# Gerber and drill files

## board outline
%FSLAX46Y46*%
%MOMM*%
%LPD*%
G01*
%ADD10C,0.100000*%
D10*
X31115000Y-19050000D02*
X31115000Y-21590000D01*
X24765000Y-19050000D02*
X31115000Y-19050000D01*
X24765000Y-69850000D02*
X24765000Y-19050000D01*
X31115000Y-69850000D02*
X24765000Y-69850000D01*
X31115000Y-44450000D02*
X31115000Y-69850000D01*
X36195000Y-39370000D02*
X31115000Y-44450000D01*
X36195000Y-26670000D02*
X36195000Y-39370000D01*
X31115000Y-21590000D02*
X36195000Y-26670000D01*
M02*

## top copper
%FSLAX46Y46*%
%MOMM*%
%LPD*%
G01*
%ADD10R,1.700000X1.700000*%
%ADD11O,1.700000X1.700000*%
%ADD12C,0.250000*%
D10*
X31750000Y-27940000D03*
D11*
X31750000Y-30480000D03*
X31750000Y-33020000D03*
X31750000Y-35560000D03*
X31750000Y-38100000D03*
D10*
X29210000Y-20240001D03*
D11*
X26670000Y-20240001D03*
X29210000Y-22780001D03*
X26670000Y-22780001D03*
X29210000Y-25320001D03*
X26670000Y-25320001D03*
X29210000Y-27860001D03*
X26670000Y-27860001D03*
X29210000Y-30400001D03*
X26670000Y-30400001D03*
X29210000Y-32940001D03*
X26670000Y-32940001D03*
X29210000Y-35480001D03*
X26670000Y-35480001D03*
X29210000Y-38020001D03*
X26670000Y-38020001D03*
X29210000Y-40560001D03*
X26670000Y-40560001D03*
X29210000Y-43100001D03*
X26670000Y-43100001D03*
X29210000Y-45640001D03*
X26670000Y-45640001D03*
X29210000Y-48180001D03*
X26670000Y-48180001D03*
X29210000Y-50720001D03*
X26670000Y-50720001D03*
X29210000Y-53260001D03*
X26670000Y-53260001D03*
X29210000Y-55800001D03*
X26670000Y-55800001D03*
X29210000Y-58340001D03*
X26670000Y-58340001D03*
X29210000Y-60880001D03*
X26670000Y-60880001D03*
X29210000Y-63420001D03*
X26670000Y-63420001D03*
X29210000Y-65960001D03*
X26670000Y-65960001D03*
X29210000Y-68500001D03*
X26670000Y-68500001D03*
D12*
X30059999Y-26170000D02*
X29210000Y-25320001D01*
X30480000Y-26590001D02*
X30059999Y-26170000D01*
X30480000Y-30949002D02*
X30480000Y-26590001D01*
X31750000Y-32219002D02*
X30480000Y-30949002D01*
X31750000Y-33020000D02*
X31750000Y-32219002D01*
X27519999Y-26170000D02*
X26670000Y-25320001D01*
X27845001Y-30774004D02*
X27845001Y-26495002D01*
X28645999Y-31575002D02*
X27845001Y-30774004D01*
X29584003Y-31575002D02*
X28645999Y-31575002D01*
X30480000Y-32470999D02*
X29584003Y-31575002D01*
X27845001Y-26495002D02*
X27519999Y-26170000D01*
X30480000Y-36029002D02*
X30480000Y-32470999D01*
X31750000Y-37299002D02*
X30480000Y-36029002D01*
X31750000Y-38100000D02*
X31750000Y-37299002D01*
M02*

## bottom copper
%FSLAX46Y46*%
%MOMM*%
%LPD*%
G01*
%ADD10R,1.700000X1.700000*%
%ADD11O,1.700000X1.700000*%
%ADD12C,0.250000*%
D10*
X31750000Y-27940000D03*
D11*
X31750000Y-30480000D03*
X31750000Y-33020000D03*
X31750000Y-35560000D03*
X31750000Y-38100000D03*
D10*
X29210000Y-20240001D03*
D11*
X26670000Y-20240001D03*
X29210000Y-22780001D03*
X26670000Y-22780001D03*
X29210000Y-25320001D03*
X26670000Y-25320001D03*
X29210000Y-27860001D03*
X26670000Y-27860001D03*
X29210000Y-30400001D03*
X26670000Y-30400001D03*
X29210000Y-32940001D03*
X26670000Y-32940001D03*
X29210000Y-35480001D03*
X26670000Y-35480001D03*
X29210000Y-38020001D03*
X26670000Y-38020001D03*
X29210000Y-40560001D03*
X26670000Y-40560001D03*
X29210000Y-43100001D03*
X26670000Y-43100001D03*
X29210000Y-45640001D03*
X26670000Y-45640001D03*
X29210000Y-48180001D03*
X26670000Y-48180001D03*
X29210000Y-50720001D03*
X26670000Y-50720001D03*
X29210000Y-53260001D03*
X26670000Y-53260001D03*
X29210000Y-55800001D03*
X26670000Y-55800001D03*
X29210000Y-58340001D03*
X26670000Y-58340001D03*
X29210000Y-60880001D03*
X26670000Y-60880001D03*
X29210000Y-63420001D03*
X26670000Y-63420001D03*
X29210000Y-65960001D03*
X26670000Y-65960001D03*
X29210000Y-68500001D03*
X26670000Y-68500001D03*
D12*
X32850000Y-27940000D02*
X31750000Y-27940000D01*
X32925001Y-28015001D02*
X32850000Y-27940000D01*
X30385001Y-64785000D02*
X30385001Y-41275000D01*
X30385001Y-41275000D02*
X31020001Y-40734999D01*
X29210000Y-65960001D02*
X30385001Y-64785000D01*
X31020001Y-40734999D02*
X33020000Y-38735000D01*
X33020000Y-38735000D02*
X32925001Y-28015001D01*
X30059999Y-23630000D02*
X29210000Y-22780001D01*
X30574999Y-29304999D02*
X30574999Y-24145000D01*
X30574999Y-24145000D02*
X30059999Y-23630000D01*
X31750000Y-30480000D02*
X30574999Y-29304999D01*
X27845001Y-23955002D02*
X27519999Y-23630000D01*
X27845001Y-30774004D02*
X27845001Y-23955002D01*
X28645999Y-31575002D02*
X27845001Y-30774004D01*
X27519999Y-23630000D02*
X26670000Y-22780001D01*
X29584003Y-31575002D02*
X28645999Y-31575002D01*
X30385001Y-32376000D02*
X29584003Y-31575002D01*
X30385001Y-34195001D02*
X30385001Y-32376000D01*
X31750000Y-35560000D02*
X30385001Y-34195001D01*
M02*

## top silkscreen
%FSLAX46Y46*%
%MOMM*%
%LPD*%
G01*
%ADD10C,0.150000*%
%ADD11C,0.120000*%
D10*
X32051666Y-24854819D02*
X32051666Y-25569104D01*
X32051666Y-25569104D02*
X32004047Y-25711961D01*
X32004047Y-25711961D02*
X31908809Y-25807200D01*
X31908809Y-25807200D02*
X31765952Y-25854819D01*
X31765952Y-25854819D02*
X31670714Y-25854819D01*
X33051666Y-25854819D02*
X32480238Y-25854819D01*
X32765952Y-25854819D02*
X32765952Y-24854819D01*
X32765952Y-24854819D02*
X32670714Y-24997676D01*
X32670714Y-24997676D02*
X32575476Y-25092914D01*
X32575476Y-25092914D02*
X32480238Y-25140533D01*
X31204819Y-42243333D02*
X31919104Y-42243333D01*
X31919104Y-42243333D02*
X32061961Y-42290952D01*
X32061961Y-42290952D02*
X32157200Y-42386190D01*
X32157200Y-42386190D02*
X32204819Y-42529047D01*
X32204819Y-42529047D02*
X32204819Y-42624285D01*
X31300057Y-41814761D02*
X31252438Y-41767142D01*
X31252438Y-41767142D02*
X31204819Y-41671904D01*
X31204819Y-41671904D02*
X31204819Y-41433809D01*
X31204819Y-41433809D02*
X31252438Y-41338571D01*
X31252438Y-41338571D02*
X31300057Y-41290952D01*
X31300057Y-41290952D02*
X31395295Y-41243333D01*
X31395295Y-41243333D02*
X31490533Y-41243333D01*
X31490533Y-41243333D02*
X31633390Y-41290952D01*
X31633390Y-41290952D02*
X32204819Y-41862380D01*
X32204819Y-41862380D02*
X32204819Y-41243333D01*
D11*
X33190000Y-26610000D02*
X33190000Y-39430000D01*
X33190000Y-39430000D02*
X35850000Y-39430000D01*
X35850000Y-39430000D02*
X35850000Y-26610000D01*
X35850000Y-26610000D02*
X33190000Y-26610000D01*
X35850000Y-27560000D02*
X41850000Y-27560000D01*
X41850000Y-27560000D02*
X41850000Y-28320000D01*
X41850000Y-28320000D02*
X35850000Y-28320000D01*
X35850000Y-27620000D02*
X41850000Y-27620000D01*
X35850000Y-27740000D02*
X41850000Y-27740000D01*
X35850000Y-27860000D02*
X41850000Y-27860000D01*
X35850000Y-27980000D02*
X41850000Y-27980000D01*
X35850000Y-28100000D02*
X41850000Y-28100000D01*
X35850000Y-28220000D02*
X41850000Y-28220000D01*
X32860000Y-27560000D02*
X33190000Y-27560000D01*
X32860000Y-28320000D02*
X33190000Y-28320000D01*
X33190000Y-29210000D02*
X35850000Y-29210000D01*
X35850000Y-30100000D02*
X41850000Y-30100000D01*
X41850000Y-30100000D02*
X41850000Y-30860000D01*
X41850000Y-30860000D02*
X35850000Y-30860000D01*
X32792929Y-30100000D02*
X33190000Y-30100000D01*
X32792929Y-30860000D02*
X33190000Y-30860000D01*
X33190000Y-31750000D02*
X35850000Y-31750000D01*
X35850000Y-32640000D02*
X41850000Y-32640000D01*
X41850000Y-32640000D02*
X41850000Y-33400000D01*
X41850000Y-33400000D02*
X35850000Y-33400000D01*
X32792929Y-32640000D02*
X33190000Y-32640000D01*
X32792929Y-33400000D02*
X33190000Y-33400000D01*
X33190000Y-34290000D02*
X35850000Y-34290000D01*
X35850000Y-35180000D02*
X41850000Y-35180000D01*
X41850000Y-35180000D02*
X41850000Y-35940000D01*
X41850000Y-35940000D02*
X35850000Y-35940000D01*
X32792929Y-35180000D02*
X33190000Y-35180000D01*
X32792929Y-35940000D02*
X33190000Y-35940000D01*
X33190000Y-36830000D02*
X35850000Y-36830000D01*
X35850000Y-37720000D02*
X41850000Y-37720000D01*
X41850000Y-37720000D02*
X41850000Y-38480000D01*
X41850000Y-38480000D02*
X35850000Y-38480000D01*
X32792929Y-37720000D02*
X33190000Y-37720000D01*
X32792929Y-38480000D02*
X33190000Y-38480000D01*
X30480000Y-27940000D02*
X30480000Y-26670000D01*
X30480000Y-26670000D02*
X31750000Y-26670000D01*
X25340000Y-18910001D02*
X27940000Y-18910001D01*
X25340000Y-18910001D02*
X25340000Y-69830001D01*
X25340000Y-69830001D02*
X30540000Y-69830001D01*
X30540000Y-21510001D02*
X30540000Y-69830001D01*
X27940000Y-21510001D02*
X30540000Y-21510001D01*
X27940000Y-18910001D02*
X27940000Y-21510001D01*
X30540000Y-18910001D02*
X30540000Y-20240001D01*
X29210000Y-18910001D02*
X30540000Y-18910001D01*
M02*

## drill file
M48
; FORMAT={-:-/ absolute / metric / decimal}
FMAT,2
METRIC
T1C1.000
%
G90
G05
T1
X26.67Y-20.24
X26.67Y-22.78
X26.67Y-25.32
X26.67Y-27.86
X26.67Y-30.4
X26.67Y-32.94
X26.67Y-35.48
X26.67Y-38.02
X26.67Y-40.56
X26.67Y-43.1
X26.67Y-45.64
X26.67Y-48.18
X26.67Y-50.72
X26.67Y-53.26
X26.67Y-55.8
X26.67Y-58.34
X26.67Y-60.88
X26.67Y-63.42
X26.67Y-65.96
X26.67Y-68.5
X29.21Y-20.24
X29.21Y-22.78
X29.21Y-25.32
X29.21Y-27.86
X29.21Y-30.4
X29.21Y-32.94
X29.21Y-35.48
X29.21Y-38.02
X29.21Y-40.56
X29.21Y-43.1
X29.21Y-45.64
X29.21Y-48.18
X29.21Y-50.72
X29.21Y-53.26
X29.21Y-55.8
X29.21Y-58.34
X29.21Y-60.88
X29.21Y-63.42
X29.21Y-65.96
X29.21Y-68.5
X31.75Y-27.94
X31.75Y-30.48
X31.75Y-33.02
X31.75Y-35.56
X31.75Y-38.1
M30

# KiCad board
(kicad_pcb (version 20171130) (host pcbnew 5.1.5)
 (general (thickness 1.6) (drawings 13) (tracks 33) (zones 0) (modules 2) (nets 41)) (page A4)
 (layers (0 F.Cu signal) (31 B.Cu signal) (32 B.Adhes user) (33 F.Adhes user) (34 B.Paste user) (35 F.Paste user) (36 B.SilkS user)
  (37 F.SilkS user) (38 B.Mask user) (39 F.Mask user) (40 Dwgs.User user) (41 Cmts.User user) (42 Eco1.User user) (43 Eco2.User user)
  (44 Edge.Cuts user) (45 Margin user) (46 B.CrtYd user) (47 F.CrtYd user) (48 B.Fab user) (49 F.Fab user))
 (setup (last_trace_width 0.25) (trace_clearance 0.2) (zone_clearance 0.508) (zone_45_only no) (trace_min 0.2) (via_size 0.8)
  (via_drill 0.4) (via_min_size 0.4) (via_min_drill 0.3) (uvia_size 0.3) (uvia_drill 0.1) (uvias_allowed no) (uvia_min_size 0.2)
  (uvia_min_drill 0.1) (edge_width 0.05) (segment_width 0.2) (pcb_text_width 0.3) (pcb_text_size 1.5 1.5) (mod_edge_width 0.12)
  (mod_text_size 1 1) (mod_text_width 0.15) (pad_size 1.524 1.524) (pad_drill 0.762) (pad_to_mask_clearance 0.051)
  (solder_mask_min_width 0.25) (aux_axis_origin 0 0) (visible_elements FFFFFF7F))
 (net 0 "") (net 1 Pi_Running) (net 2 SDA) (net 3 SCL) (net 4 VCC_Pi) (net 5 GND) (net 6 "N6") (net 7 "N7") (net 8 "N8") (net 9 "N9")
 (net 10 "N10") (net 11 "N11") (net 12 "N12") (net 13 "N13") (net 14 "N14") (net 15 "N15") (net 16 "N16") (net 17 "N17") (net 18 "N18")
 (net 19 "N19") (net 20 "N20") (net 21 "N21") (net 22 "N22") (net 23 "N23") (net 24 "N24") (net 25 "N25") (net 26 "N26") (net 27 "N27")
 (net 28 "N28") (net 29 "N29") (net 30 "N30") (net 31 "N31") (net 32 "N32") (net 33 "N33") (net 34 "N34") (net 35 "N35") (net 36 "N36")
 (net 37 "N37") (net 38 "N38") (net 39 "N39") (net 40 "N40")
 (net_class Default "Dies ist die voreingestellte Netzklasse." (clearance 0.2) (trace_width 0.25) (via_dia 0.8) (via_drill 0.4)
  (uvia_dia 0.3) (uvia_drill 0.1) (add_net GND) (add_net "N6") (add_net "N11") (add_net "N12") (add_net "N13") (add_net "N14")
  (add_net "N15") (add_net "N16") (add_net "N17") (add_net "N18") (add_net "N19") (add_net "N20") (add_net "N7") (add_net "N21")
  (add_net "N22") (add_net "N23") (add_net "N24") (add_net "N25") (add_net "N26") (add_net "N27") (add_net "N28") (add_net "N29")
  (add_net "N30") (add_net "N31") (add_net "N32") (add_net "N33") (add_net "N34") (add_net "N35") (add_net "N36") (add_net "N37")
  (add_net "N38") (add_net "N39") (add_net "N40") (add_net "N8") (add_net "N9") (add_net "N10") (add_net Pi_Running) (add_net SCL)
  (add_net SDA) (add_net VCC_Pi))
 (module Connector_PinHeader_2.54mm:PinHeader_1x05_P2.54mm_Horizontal (layer F.Cu) (at 31.75 27.94)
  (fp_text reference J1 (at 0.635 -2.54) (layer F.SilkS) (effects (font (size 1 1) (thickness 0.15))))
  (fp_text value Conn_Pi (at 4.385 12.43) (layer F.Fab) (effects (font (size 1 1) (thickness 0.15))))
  (fp_line (start 1.44 -1.33) (end 1.44 11.49) (layer F.SilkS) (width 0.12))
  (fp_line (start 1.44 11.49) (end 4.1 11.49) (layer F.SilkS) (width 0.12))
  (fp_line (start 4.1 11.49) (end 4.1 -1.33) (layer F.SilkS) (width 0.12))
  (fp_line (start 4.1 -1.33) (end 1.44 -1.33) (layer F.SilkS) (width 0.12))
  (fp_line (start 4.1 -0.38) (end 10.1 -0.38) (layer F.SilkS) (width 0.12))
  (fp_line (start 10.1 -0.38) (end 10.1 0.38) (layer F.SilkS) (width 0.12))
  (fp_line (start 10.1 0.38) (end 4.1 0.38) (layer F.SilkS) (width 0.12))
  (fp_line (start 4.1 -0.32) (end 10.1 -0.32) (layer F.SilkS) (width 0.12))
  (fp_line (start 4.1 -0.2) (end 10.1 -0.2) (layer F.SilkS) (width 0.12))
  (fp_line (start 4.1 -0.08) (end 10.1 -0.08) (layer F.SilkS) (width 0.12))
  (fp_line (start 4.1 0.04) (end 10.1 0.04) (layer F.SilkS) (width 0.12))
  (fp_line (start 4.1 0.16) (end 10.1 0.16) (layer F.SilkS) (width 0.12))
  (fp_line (start 4.1 0.28) (end 10.1 0.28) (layer F.SilkS) (width 0.12))
  (fp_line (start 1.11 -0.38) (end 1.44 -0.38) (layer F.SilkS) (width 0.12))
  (fp_line (start 1.11 0.38) (end 1.44 0.38) (layer F.SilkS) (width 0.12))
  (fp_line (start 1.44 1.27) (end 4.1 1.27) (layer F.SilkS) (width 0.12))
  (fp_line (start 4.1 2.16) (end 10.1 2.16) (layer F.SilkS) (width 0.12))
  (fp_line (start 10.1 2.16) (end 10.1 2.92) (layer F.SilkS) (width 0.12))
  (fp_line (start 10.1 2.92) (end 4.1 2.92) (layer F.SilkS) (width 0.12))
  (fp_line (start 1.042929 2.16) (end 1.44 2.16) (layer F.SilkS) (width 0.12))
  (fp_line (start 1.042929 2.92) (end 1.44 2.92) (layer F.SilkS) (width 0.12))
  (fp_line (start 1.44 3.81) (end 4.1 3.81) (layer F.SilkS) (width 0.12))
  (fp_line (start 4.1 4.7) (end 10.1 4.7) (layer F.SilkS) (width 0.12))
  (fp_line (start 10.1 4.7) (end 10.1 5.46) (layer F.SilkS) (width 0.12))
  (fp_line (start 10.1 5.46) (end 4.1 5.46) (layer F.SilkS) (width 0.12))
  (fp_line (start 1.042929 4.7) (end 1.44 4.7) (layer F.SilkS) (width 0.12))
  (fp_line (start 1.042929 5.46) (end 1.44 5.46) (layer F.SilkS) (width 0.12))
  (fp_line (start 1.44 6.35) (end 4.1 6.35) (layer F.SilkS) (width 0.12))
  (fp_line (start 4.1 7.24) (end 10.1 7.24) (layer F.SilkS) (width 0.12))
  (fp_line (start 10.1 7.24) (end 10.1 8) (layer F.SilkS) (width 0.12))
  (fp_line (start 10.1 8) (end 4.1 8) (layer F.SilkS) (width 0.12))
  (fp_line (start 1.042929 7.24) (end 1.44 7.24) (layer F.SilkS) (width 0.12))
  (fp_line (start 1.042929 8) (end 1.44 8) (layer F.SilkS) (width 0.12))
  (fp_line (start 1.44 8.89) (end 4.1 8.89) (layer F.SilkS) (width 0.12))
  (fp_line (start 4.1 9.78) (end 10.1 9.78) (layer F.SilkS) (width 0.12))
  (fp_line (start 10.1 9.78) (end 10.1 10.54) (layer F.SilkS) (width 0.12))
  (fp_line (start 10.1 10.54) (end 4.1 10.54) (layer F.SilkS) (width 0.12))
  (fp_line (start 1.042929 9.78) (end 1.44 9.78) (layer F.SilkS) (width 0.12))
  (fp_line (start 1.042929 10.54) (end 1.44 10.54) (layer F.SilkS) (width 0.12))
  (fp_line (start -1.27 0) (end -1.27 -1.27) (layer F.SilkS) (width 0.12))
  (fp_line (start -1.27 -1.27) (end 0 -1.27) (layer F.SilkS) (width 0.12))
  (pad 1 thru_hole rect (at 0 0) (size 1.7 1.7) (drill 1) (layers *.Cu *.Mask) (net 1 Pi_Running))
  (pad 2 thru_hole oval (at 0 2.54) (size 1.7 1.7) (drill 1) (layers *.Cu *.Mask) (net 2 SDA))
  (pad 3 thru_hole oval (at 0 5.08) (size 1.7 1.7) (drill 1) (layers *.Cu *.Mask) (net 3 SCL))
  (pad 4 thru_hole oval (at 0 7.62) (size 1.7 1.7) (drill 1) (layers *.Cu *.Mask) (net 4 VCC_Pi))
  (pad 5 thru_hole oval (at 0 10.16) (size 1.7 1.7) (drill 1) (layers *.Cu *.Mask) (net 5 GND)))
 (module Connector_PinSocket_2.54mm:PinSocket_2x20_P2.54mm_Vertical (layer F.Cu) (at 29.21 20.240001)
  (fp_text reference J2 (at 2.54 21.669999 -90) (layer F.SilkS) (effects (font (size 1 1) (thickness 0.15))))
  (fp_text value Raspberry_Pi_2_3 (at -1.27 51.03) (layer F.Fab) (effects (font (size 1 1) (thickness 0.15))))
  (fp_line (start -3.87 -1.33) (end -1.27 -1.33) (layer F.SilkS) (width 0.12))
  (fp_line (start -3.87 -1.33) (end -3.87 49.59) (layer F.SilkS) (width 0.12))
  (fp_line (start -3.87 49.59) (end 1.33 49.59) (layer F.SilkS) (width 0.12))
  (fp_line (start 1.33 1.27) (end 1.33 49.59) (layer F.SilkS) (width 0.12))
  (fp_line (start -1.27 1.27) (end 1.33 1.27) (layer F.SilkS) (width 0.12))
  (fp_line (start -1.27 -1.33) (end -1.27 1.27) (layer F.SilkS) (width 0.12))
  (fp_line (start 1.33 -1.33) (end 1.33 0) (layer F.SilkS) (width 0.12))
  (fp_line (start 0 -1.33) (end 1.33 -1.33) (layer F.SilkS) (width 0.12))
  (pad 1 thru_hole rect (at 0 0) (size 1.7 1.7) (drill 1) (layers *.Cu *.Mask) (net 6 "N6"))
  (pad 2 thru_hole oval (at -2.54 0) (size 1.7 1.7) (drill 1) (layers *.Cu *.Mask) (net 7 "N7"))
  (pad 3 thru_hole oval (at 0 2.54) (size 1.7 1.7) (drill 1) (layers *.Cu *.Mask) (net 2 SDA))
  (pad 4 thru_hole oval (at -2.54 2.54) (size 1.7 1.7) (drill 1) (layers *.Cu *.Mask) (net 4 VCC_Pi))
  (pad 5 thru_hole oval (at 0 5.08) (size 1.7 1.7) (drill 1) (layers *.Cu *.Mask) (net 3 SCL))
  (pad 6 thru_hole oval (at -2.54 5.08) (size 1.7 1.7) (drill 1) (layers *.Cu *.Mask) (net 5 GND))
  (pad 7 thru_hole oval (at 0 7.62) (size 1.7 1.7) (drill 1) (layers *.Cu *.Mask) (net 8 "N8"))
  (pad 8 thru_hole oval (at -2.54 7.62) (size 1.7 1.7) (drill 1) (layers *.Cu *.Mask) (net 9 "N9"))
  (pad 9 thru_hole oval (at 0 10.16) (size 1.7 1.7) (drill 1) (layers *.Cu *.Mask) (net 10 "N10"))
  (pad 10 thru_hole oval (at -2.54 10.16) (size 1.7 1.7) (drill 1) (layers *.Cu *.Mask) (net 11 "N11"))
  (pad 11 thru_hole oval (at 0 12.7) (size 1.7 1.7) (drill 1) (layers *.Cu *.Mask) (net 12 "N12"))
  (pad 12 thru_hole oval (at -2.54 12.7) (size 1.7 1.7) (drill 1) (layers *.Cu *.Mask) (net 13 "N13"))
  (pad 13 thru_hole oval (at 0 15.24) (size 1.7 1.7) (drill 1) (layers *.Cu *.Mask) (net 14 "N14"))
  (pad 14 thru_hole oval (at -2.54 15.24) (size 1.7 1.7) (drill 1) (layers *.Cu *.Mask) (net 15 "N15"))
  (pad 15 thru_hole oval (at 0 17.78) (size 1.7 1.7) (drill 1) (layers *.Cu *.Mask) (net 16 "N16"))
  (pad 16 thru_hole oval (at -2.54 17.78) (size 1.7 1.7) (drill 1) (layers *.Cu *.Mask) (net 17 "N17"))
  (pad 17 thru_hole oval (at 0 20.32) (size 1.7 1.7) (drill 1) (layers *.Cu *.Mask) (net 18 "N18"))
  (pad 18 thru_hole oval (at -2.54 20.32) (size 1.7 1.7) (drill 1) (layers *.Cu *.Mask) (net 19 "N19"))
  (pad 19 thru_hole oval (at 0 22.86) (size 1.7 1.7) (drill 1) (layers *.Cu *.Mask) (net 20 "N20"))
  (pad 20 thru_hole oval (at -2.54 22.86) (size 1.7 1.7) (drill 1) (layers *.Cu *.Mask) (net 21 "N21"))
  (pad 21 thru_hole oval (at 0 25.4) (size 1.7 1.7) (drill 1) (layers *.Cu *.Mask) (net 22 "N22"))
  (pad 22 thru_hole oval (at -2.54 25.4) (size 1.7 1.7) (drill 1) (layers *.Cu *.Mask) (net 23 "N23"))
  (pad 23 thru_hole oval (at 0 27.94) (size 1.7 1.7) (drill 1) (layers *.Cu *.Mask) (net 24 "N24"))
  (pad 24 thru_hole oval (at -2.54 27.94) (size 1.7 1.7) (drill 1) (layers *.Cu *.Mask) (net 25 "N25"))
  (pad 25 thru_hole oval (at 0 30.48) (size 1.7 1.7) (drill 1) (layers *.Cu *.Mask) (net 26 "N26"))
  (pad 26 thru_hole oval (at -2.54 30.48) (size 1.7 1.7) (drill 1) (layers *.Cu *.Mask) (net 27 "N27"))
  (pad 27 thru_hole oval (at 0 33.02) (size 1.7 1.7) (drill 1) (layers *.Cu *.Mask) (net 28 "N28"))
  (pad 28 thru_hole oval (at -2.54 33.02) (size 1.7 1.7) (drill 1) (layers *.Cu *.Mask) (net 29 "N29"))
  (pad 29 thru_hole oval (at 0 35.56) (size 1.7 1.7) (drill 1) (layers *.Cu *.Mask) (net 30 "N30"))
  (pad 30 thru_hole oval (at -2.54 35.56) (size 1.7 1.7) (drill 1) (layers *.Cu *.Mask) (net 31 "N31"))
  (pad 31 thru_hole oval (at 0 38.1) (size 1.7 1.7) (drill 1) (layers *.Cu *.Mask) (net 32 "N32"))
  (pad 32 thru_hole oval (at -2.54 38.1) (size 1.7 1.7) (drill 1) (layers *.Cu *.Mask) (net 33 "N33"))
  (pad 33 thru_hole oval (at 0 40.64) (size 1.7 1.7) (drill 1) (layers *.Cu *.Mask) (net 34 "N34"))
  (pad 34 thru_hole oval (at -2.54 40.64) (size 1.7 1.7) (drill 1) (layers *.Cu *.Mask) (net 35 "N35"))
  (pad 35 thru_hole oval (at 0 43.18) (size 1.7 1.7) (drill 1) (layers *.Cu *.Mask) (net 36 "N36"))
  (pad 36 thru_hole oval (at -2.54 43.18) (size 1.7 1.7) (drill 1) (layers *.Cu *.Mask) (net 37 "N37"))
  (pad 37 thru_hole oval (at 0 45.72) (size 1.7 1.7) (drill 1) (layers *.Cu *.Mask) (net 1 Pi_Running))
  (pad 38 thru_hole oval (at -2.54 45.72) (size 1.7 1.7) (drill 1) (layers *.Cu *.Mask) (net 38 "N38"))
  (pad 39 thru_hole oval (at 0 48.26) (size 1.7 1.7) (drill 1) (layers *.Cu *.Mask) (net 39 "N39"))
  (pad 40 thru_hole oval (at -2.54 48.26) (size 1.7 1.7) (drill 1) (layers *.Cu *.Mask) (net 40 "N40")))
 (gr_line (start 31.115 19.05) (end 31.115 21.59) (layer Edge.Cuts) (width 0.1))
 (gr_line (start 24.765 19.05) (end 31.115 19.05) (layer Edge.Cuts) (width 0.1))
 (gr_line (start 24.765 69.85) (end 24.765 19.05) (layer Edge.Cuts) (width 0.1))
 (gr_line (start 31.115 69.85) (end 24.765 69.85) (layer Edge.Cuts) (width 0.1))
 (gr_line (start 31.115 44.45) (end 31.115 69.85) (layer Edge.Cuts) (width 0.1))
 (gr_line (start 36.195 39.37) (end 31.115 44.45) (layer Edge.Cuts) (width 0.1))
 (gr_line (start 36.195 26.67) (end 36.195 39.37) (layer Edge.Cuts) (width 0.1))
 (gr_line (start 31.115 21.59) (end 36.195 26.67) (layer Edge.Cuts) (width 0.1))
 (segment (start 32.85 27.94) (end 31.75 27.94) (width 0.25) (layer B.Cu) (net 1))
 (segment (start 32.925001 28.015001) (end 32.85 27.94) (width 0.25) (layer B.Cu) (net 1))
 (segment (start 30.385001 64.785) (end 30.385001 41.275) (width 0.25) (layer B.Cu) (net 1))
 (segment (start 30.385001 41.275) (end 31.020001 40.734999) (width 0.25) (layer B.Cu) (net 1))
 (segment (start 29.21 65.960001) (end 30.385001 64.785) (width 0.25) (layer B.Cu) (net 1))
 (segment (start 31.020001 40.734999) (end 33.02 38.735) (width 0.25) (layer B.Cu) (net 1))
 (segment (start 33.02 38.735) (end 32.925001 28.015001) (width 0.25) (layer B.Cu) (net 1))
 (segment (start 30.059999 23.63) (end 29.21 22.780001) (width 0.25) (layer B.Cu) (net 2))
 (segment (start 30.574999 29.304999) (end 30.574999 24.145) (width 0.25) (layer B.Cu) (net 2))
 (segment (start 30.574999 24.145) (end 30.059999 23.63) (width 0.25) (layer B.Cu) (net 2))
 (segment (start 31.75 30.48) (end 30.574999 29.304999) (width 0.25) (layer B.Cu) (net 2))
 (segment (start 30.059999 26.17) (end 29.21 25.320001) (width 0.25) (layer F.Cu) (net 3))
 (segment (start 30.48 26.590001) (end 30.059999 26.17) (width 0.25) (layer F.Cu) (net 3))
 (segment (start 30.48 30.949002) (end 30.48 26.590001) (width 0.25) (layer F.Cu) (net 3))
 (segment (start 31.75 32.219002) (end 30.48 30.949002) (width 0.25) (layer F.Cu) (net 3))
 (segment (start 31.75 33.02) (end 31.75 32.219002) (width 0.25) (layer F.Cu) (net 3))
 (segment (start 27.845001 23.955002) (end 27.519999 23.63) (width 0.25) (layer B.Cu) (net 4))
 (segment (start 27.845001 30.774004) (end 27.845001 23.955002) (width 0.25) (layer B.Cu) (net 4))
 (segment (start 28.645999 31.575002) (end 27.845001 30.774004) (width 0.25) (layer B.Cu) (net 4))
 (segment (start 27.519999 23.63) (end 26.67 22.780001) (width 0.25) (layer B.Cu) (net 4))
 (segment (start 29.584003 31.575002) (end 28.645999 31.575002) (width 0.25) (layer B.Cu) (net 4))
 (segment (start 30.385001 32.376) (end 29.584003 31.575002) (width 0.25) (layer B.Cu) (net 4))
 (segment (start 30.385001 34.195001) (end 30.385001 32.376) (width 0.25) (layer B.Cu) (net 4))
 (segment (start 31.75 35.56) (end 30.385001 34.195001) (width 0.25) (layer B.Cu) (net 4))
 (segment (start 27.519999 26.17) (end 26.67 25.320001) (width 0.25) (layer F.Cu) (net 5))
 (segment (start 27.845001 30.774004) (end 27.845001 26.495002) (width 0.25) (layer F.Cu) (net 5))
 (segment (start 28.645999 31.575002) (end 27.845001 30.774004) (width 0.25) (layer F.Cu) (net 5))
 (segment (start 29.584003 31.575002) (end 28.645999 31.575002) (width 0.25) (layer F.Cu) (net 5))
 (segment (start 30.48 32.470999) (end 29.584003 31.575002) (width 0.25) (layer F.Cu) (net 5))
 (segment (start 27.845001 26.495002) (end 27.519999 26.17) (width 0.25) (layer F.Cu) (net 5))
 (segment (start 30.48 36.029002) (end 30.48 32.470999) (width 0.25) (layer F.Cu) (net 5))
 (segment (start 31.75 37.299002) (end 30.48 36.029002) (width 0.25) (layer F.Cu) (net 5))
 (segment (start 31.75 38.1) (end 31.75 37.299002) (width 0.25) (layer F.Cu) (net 5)))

